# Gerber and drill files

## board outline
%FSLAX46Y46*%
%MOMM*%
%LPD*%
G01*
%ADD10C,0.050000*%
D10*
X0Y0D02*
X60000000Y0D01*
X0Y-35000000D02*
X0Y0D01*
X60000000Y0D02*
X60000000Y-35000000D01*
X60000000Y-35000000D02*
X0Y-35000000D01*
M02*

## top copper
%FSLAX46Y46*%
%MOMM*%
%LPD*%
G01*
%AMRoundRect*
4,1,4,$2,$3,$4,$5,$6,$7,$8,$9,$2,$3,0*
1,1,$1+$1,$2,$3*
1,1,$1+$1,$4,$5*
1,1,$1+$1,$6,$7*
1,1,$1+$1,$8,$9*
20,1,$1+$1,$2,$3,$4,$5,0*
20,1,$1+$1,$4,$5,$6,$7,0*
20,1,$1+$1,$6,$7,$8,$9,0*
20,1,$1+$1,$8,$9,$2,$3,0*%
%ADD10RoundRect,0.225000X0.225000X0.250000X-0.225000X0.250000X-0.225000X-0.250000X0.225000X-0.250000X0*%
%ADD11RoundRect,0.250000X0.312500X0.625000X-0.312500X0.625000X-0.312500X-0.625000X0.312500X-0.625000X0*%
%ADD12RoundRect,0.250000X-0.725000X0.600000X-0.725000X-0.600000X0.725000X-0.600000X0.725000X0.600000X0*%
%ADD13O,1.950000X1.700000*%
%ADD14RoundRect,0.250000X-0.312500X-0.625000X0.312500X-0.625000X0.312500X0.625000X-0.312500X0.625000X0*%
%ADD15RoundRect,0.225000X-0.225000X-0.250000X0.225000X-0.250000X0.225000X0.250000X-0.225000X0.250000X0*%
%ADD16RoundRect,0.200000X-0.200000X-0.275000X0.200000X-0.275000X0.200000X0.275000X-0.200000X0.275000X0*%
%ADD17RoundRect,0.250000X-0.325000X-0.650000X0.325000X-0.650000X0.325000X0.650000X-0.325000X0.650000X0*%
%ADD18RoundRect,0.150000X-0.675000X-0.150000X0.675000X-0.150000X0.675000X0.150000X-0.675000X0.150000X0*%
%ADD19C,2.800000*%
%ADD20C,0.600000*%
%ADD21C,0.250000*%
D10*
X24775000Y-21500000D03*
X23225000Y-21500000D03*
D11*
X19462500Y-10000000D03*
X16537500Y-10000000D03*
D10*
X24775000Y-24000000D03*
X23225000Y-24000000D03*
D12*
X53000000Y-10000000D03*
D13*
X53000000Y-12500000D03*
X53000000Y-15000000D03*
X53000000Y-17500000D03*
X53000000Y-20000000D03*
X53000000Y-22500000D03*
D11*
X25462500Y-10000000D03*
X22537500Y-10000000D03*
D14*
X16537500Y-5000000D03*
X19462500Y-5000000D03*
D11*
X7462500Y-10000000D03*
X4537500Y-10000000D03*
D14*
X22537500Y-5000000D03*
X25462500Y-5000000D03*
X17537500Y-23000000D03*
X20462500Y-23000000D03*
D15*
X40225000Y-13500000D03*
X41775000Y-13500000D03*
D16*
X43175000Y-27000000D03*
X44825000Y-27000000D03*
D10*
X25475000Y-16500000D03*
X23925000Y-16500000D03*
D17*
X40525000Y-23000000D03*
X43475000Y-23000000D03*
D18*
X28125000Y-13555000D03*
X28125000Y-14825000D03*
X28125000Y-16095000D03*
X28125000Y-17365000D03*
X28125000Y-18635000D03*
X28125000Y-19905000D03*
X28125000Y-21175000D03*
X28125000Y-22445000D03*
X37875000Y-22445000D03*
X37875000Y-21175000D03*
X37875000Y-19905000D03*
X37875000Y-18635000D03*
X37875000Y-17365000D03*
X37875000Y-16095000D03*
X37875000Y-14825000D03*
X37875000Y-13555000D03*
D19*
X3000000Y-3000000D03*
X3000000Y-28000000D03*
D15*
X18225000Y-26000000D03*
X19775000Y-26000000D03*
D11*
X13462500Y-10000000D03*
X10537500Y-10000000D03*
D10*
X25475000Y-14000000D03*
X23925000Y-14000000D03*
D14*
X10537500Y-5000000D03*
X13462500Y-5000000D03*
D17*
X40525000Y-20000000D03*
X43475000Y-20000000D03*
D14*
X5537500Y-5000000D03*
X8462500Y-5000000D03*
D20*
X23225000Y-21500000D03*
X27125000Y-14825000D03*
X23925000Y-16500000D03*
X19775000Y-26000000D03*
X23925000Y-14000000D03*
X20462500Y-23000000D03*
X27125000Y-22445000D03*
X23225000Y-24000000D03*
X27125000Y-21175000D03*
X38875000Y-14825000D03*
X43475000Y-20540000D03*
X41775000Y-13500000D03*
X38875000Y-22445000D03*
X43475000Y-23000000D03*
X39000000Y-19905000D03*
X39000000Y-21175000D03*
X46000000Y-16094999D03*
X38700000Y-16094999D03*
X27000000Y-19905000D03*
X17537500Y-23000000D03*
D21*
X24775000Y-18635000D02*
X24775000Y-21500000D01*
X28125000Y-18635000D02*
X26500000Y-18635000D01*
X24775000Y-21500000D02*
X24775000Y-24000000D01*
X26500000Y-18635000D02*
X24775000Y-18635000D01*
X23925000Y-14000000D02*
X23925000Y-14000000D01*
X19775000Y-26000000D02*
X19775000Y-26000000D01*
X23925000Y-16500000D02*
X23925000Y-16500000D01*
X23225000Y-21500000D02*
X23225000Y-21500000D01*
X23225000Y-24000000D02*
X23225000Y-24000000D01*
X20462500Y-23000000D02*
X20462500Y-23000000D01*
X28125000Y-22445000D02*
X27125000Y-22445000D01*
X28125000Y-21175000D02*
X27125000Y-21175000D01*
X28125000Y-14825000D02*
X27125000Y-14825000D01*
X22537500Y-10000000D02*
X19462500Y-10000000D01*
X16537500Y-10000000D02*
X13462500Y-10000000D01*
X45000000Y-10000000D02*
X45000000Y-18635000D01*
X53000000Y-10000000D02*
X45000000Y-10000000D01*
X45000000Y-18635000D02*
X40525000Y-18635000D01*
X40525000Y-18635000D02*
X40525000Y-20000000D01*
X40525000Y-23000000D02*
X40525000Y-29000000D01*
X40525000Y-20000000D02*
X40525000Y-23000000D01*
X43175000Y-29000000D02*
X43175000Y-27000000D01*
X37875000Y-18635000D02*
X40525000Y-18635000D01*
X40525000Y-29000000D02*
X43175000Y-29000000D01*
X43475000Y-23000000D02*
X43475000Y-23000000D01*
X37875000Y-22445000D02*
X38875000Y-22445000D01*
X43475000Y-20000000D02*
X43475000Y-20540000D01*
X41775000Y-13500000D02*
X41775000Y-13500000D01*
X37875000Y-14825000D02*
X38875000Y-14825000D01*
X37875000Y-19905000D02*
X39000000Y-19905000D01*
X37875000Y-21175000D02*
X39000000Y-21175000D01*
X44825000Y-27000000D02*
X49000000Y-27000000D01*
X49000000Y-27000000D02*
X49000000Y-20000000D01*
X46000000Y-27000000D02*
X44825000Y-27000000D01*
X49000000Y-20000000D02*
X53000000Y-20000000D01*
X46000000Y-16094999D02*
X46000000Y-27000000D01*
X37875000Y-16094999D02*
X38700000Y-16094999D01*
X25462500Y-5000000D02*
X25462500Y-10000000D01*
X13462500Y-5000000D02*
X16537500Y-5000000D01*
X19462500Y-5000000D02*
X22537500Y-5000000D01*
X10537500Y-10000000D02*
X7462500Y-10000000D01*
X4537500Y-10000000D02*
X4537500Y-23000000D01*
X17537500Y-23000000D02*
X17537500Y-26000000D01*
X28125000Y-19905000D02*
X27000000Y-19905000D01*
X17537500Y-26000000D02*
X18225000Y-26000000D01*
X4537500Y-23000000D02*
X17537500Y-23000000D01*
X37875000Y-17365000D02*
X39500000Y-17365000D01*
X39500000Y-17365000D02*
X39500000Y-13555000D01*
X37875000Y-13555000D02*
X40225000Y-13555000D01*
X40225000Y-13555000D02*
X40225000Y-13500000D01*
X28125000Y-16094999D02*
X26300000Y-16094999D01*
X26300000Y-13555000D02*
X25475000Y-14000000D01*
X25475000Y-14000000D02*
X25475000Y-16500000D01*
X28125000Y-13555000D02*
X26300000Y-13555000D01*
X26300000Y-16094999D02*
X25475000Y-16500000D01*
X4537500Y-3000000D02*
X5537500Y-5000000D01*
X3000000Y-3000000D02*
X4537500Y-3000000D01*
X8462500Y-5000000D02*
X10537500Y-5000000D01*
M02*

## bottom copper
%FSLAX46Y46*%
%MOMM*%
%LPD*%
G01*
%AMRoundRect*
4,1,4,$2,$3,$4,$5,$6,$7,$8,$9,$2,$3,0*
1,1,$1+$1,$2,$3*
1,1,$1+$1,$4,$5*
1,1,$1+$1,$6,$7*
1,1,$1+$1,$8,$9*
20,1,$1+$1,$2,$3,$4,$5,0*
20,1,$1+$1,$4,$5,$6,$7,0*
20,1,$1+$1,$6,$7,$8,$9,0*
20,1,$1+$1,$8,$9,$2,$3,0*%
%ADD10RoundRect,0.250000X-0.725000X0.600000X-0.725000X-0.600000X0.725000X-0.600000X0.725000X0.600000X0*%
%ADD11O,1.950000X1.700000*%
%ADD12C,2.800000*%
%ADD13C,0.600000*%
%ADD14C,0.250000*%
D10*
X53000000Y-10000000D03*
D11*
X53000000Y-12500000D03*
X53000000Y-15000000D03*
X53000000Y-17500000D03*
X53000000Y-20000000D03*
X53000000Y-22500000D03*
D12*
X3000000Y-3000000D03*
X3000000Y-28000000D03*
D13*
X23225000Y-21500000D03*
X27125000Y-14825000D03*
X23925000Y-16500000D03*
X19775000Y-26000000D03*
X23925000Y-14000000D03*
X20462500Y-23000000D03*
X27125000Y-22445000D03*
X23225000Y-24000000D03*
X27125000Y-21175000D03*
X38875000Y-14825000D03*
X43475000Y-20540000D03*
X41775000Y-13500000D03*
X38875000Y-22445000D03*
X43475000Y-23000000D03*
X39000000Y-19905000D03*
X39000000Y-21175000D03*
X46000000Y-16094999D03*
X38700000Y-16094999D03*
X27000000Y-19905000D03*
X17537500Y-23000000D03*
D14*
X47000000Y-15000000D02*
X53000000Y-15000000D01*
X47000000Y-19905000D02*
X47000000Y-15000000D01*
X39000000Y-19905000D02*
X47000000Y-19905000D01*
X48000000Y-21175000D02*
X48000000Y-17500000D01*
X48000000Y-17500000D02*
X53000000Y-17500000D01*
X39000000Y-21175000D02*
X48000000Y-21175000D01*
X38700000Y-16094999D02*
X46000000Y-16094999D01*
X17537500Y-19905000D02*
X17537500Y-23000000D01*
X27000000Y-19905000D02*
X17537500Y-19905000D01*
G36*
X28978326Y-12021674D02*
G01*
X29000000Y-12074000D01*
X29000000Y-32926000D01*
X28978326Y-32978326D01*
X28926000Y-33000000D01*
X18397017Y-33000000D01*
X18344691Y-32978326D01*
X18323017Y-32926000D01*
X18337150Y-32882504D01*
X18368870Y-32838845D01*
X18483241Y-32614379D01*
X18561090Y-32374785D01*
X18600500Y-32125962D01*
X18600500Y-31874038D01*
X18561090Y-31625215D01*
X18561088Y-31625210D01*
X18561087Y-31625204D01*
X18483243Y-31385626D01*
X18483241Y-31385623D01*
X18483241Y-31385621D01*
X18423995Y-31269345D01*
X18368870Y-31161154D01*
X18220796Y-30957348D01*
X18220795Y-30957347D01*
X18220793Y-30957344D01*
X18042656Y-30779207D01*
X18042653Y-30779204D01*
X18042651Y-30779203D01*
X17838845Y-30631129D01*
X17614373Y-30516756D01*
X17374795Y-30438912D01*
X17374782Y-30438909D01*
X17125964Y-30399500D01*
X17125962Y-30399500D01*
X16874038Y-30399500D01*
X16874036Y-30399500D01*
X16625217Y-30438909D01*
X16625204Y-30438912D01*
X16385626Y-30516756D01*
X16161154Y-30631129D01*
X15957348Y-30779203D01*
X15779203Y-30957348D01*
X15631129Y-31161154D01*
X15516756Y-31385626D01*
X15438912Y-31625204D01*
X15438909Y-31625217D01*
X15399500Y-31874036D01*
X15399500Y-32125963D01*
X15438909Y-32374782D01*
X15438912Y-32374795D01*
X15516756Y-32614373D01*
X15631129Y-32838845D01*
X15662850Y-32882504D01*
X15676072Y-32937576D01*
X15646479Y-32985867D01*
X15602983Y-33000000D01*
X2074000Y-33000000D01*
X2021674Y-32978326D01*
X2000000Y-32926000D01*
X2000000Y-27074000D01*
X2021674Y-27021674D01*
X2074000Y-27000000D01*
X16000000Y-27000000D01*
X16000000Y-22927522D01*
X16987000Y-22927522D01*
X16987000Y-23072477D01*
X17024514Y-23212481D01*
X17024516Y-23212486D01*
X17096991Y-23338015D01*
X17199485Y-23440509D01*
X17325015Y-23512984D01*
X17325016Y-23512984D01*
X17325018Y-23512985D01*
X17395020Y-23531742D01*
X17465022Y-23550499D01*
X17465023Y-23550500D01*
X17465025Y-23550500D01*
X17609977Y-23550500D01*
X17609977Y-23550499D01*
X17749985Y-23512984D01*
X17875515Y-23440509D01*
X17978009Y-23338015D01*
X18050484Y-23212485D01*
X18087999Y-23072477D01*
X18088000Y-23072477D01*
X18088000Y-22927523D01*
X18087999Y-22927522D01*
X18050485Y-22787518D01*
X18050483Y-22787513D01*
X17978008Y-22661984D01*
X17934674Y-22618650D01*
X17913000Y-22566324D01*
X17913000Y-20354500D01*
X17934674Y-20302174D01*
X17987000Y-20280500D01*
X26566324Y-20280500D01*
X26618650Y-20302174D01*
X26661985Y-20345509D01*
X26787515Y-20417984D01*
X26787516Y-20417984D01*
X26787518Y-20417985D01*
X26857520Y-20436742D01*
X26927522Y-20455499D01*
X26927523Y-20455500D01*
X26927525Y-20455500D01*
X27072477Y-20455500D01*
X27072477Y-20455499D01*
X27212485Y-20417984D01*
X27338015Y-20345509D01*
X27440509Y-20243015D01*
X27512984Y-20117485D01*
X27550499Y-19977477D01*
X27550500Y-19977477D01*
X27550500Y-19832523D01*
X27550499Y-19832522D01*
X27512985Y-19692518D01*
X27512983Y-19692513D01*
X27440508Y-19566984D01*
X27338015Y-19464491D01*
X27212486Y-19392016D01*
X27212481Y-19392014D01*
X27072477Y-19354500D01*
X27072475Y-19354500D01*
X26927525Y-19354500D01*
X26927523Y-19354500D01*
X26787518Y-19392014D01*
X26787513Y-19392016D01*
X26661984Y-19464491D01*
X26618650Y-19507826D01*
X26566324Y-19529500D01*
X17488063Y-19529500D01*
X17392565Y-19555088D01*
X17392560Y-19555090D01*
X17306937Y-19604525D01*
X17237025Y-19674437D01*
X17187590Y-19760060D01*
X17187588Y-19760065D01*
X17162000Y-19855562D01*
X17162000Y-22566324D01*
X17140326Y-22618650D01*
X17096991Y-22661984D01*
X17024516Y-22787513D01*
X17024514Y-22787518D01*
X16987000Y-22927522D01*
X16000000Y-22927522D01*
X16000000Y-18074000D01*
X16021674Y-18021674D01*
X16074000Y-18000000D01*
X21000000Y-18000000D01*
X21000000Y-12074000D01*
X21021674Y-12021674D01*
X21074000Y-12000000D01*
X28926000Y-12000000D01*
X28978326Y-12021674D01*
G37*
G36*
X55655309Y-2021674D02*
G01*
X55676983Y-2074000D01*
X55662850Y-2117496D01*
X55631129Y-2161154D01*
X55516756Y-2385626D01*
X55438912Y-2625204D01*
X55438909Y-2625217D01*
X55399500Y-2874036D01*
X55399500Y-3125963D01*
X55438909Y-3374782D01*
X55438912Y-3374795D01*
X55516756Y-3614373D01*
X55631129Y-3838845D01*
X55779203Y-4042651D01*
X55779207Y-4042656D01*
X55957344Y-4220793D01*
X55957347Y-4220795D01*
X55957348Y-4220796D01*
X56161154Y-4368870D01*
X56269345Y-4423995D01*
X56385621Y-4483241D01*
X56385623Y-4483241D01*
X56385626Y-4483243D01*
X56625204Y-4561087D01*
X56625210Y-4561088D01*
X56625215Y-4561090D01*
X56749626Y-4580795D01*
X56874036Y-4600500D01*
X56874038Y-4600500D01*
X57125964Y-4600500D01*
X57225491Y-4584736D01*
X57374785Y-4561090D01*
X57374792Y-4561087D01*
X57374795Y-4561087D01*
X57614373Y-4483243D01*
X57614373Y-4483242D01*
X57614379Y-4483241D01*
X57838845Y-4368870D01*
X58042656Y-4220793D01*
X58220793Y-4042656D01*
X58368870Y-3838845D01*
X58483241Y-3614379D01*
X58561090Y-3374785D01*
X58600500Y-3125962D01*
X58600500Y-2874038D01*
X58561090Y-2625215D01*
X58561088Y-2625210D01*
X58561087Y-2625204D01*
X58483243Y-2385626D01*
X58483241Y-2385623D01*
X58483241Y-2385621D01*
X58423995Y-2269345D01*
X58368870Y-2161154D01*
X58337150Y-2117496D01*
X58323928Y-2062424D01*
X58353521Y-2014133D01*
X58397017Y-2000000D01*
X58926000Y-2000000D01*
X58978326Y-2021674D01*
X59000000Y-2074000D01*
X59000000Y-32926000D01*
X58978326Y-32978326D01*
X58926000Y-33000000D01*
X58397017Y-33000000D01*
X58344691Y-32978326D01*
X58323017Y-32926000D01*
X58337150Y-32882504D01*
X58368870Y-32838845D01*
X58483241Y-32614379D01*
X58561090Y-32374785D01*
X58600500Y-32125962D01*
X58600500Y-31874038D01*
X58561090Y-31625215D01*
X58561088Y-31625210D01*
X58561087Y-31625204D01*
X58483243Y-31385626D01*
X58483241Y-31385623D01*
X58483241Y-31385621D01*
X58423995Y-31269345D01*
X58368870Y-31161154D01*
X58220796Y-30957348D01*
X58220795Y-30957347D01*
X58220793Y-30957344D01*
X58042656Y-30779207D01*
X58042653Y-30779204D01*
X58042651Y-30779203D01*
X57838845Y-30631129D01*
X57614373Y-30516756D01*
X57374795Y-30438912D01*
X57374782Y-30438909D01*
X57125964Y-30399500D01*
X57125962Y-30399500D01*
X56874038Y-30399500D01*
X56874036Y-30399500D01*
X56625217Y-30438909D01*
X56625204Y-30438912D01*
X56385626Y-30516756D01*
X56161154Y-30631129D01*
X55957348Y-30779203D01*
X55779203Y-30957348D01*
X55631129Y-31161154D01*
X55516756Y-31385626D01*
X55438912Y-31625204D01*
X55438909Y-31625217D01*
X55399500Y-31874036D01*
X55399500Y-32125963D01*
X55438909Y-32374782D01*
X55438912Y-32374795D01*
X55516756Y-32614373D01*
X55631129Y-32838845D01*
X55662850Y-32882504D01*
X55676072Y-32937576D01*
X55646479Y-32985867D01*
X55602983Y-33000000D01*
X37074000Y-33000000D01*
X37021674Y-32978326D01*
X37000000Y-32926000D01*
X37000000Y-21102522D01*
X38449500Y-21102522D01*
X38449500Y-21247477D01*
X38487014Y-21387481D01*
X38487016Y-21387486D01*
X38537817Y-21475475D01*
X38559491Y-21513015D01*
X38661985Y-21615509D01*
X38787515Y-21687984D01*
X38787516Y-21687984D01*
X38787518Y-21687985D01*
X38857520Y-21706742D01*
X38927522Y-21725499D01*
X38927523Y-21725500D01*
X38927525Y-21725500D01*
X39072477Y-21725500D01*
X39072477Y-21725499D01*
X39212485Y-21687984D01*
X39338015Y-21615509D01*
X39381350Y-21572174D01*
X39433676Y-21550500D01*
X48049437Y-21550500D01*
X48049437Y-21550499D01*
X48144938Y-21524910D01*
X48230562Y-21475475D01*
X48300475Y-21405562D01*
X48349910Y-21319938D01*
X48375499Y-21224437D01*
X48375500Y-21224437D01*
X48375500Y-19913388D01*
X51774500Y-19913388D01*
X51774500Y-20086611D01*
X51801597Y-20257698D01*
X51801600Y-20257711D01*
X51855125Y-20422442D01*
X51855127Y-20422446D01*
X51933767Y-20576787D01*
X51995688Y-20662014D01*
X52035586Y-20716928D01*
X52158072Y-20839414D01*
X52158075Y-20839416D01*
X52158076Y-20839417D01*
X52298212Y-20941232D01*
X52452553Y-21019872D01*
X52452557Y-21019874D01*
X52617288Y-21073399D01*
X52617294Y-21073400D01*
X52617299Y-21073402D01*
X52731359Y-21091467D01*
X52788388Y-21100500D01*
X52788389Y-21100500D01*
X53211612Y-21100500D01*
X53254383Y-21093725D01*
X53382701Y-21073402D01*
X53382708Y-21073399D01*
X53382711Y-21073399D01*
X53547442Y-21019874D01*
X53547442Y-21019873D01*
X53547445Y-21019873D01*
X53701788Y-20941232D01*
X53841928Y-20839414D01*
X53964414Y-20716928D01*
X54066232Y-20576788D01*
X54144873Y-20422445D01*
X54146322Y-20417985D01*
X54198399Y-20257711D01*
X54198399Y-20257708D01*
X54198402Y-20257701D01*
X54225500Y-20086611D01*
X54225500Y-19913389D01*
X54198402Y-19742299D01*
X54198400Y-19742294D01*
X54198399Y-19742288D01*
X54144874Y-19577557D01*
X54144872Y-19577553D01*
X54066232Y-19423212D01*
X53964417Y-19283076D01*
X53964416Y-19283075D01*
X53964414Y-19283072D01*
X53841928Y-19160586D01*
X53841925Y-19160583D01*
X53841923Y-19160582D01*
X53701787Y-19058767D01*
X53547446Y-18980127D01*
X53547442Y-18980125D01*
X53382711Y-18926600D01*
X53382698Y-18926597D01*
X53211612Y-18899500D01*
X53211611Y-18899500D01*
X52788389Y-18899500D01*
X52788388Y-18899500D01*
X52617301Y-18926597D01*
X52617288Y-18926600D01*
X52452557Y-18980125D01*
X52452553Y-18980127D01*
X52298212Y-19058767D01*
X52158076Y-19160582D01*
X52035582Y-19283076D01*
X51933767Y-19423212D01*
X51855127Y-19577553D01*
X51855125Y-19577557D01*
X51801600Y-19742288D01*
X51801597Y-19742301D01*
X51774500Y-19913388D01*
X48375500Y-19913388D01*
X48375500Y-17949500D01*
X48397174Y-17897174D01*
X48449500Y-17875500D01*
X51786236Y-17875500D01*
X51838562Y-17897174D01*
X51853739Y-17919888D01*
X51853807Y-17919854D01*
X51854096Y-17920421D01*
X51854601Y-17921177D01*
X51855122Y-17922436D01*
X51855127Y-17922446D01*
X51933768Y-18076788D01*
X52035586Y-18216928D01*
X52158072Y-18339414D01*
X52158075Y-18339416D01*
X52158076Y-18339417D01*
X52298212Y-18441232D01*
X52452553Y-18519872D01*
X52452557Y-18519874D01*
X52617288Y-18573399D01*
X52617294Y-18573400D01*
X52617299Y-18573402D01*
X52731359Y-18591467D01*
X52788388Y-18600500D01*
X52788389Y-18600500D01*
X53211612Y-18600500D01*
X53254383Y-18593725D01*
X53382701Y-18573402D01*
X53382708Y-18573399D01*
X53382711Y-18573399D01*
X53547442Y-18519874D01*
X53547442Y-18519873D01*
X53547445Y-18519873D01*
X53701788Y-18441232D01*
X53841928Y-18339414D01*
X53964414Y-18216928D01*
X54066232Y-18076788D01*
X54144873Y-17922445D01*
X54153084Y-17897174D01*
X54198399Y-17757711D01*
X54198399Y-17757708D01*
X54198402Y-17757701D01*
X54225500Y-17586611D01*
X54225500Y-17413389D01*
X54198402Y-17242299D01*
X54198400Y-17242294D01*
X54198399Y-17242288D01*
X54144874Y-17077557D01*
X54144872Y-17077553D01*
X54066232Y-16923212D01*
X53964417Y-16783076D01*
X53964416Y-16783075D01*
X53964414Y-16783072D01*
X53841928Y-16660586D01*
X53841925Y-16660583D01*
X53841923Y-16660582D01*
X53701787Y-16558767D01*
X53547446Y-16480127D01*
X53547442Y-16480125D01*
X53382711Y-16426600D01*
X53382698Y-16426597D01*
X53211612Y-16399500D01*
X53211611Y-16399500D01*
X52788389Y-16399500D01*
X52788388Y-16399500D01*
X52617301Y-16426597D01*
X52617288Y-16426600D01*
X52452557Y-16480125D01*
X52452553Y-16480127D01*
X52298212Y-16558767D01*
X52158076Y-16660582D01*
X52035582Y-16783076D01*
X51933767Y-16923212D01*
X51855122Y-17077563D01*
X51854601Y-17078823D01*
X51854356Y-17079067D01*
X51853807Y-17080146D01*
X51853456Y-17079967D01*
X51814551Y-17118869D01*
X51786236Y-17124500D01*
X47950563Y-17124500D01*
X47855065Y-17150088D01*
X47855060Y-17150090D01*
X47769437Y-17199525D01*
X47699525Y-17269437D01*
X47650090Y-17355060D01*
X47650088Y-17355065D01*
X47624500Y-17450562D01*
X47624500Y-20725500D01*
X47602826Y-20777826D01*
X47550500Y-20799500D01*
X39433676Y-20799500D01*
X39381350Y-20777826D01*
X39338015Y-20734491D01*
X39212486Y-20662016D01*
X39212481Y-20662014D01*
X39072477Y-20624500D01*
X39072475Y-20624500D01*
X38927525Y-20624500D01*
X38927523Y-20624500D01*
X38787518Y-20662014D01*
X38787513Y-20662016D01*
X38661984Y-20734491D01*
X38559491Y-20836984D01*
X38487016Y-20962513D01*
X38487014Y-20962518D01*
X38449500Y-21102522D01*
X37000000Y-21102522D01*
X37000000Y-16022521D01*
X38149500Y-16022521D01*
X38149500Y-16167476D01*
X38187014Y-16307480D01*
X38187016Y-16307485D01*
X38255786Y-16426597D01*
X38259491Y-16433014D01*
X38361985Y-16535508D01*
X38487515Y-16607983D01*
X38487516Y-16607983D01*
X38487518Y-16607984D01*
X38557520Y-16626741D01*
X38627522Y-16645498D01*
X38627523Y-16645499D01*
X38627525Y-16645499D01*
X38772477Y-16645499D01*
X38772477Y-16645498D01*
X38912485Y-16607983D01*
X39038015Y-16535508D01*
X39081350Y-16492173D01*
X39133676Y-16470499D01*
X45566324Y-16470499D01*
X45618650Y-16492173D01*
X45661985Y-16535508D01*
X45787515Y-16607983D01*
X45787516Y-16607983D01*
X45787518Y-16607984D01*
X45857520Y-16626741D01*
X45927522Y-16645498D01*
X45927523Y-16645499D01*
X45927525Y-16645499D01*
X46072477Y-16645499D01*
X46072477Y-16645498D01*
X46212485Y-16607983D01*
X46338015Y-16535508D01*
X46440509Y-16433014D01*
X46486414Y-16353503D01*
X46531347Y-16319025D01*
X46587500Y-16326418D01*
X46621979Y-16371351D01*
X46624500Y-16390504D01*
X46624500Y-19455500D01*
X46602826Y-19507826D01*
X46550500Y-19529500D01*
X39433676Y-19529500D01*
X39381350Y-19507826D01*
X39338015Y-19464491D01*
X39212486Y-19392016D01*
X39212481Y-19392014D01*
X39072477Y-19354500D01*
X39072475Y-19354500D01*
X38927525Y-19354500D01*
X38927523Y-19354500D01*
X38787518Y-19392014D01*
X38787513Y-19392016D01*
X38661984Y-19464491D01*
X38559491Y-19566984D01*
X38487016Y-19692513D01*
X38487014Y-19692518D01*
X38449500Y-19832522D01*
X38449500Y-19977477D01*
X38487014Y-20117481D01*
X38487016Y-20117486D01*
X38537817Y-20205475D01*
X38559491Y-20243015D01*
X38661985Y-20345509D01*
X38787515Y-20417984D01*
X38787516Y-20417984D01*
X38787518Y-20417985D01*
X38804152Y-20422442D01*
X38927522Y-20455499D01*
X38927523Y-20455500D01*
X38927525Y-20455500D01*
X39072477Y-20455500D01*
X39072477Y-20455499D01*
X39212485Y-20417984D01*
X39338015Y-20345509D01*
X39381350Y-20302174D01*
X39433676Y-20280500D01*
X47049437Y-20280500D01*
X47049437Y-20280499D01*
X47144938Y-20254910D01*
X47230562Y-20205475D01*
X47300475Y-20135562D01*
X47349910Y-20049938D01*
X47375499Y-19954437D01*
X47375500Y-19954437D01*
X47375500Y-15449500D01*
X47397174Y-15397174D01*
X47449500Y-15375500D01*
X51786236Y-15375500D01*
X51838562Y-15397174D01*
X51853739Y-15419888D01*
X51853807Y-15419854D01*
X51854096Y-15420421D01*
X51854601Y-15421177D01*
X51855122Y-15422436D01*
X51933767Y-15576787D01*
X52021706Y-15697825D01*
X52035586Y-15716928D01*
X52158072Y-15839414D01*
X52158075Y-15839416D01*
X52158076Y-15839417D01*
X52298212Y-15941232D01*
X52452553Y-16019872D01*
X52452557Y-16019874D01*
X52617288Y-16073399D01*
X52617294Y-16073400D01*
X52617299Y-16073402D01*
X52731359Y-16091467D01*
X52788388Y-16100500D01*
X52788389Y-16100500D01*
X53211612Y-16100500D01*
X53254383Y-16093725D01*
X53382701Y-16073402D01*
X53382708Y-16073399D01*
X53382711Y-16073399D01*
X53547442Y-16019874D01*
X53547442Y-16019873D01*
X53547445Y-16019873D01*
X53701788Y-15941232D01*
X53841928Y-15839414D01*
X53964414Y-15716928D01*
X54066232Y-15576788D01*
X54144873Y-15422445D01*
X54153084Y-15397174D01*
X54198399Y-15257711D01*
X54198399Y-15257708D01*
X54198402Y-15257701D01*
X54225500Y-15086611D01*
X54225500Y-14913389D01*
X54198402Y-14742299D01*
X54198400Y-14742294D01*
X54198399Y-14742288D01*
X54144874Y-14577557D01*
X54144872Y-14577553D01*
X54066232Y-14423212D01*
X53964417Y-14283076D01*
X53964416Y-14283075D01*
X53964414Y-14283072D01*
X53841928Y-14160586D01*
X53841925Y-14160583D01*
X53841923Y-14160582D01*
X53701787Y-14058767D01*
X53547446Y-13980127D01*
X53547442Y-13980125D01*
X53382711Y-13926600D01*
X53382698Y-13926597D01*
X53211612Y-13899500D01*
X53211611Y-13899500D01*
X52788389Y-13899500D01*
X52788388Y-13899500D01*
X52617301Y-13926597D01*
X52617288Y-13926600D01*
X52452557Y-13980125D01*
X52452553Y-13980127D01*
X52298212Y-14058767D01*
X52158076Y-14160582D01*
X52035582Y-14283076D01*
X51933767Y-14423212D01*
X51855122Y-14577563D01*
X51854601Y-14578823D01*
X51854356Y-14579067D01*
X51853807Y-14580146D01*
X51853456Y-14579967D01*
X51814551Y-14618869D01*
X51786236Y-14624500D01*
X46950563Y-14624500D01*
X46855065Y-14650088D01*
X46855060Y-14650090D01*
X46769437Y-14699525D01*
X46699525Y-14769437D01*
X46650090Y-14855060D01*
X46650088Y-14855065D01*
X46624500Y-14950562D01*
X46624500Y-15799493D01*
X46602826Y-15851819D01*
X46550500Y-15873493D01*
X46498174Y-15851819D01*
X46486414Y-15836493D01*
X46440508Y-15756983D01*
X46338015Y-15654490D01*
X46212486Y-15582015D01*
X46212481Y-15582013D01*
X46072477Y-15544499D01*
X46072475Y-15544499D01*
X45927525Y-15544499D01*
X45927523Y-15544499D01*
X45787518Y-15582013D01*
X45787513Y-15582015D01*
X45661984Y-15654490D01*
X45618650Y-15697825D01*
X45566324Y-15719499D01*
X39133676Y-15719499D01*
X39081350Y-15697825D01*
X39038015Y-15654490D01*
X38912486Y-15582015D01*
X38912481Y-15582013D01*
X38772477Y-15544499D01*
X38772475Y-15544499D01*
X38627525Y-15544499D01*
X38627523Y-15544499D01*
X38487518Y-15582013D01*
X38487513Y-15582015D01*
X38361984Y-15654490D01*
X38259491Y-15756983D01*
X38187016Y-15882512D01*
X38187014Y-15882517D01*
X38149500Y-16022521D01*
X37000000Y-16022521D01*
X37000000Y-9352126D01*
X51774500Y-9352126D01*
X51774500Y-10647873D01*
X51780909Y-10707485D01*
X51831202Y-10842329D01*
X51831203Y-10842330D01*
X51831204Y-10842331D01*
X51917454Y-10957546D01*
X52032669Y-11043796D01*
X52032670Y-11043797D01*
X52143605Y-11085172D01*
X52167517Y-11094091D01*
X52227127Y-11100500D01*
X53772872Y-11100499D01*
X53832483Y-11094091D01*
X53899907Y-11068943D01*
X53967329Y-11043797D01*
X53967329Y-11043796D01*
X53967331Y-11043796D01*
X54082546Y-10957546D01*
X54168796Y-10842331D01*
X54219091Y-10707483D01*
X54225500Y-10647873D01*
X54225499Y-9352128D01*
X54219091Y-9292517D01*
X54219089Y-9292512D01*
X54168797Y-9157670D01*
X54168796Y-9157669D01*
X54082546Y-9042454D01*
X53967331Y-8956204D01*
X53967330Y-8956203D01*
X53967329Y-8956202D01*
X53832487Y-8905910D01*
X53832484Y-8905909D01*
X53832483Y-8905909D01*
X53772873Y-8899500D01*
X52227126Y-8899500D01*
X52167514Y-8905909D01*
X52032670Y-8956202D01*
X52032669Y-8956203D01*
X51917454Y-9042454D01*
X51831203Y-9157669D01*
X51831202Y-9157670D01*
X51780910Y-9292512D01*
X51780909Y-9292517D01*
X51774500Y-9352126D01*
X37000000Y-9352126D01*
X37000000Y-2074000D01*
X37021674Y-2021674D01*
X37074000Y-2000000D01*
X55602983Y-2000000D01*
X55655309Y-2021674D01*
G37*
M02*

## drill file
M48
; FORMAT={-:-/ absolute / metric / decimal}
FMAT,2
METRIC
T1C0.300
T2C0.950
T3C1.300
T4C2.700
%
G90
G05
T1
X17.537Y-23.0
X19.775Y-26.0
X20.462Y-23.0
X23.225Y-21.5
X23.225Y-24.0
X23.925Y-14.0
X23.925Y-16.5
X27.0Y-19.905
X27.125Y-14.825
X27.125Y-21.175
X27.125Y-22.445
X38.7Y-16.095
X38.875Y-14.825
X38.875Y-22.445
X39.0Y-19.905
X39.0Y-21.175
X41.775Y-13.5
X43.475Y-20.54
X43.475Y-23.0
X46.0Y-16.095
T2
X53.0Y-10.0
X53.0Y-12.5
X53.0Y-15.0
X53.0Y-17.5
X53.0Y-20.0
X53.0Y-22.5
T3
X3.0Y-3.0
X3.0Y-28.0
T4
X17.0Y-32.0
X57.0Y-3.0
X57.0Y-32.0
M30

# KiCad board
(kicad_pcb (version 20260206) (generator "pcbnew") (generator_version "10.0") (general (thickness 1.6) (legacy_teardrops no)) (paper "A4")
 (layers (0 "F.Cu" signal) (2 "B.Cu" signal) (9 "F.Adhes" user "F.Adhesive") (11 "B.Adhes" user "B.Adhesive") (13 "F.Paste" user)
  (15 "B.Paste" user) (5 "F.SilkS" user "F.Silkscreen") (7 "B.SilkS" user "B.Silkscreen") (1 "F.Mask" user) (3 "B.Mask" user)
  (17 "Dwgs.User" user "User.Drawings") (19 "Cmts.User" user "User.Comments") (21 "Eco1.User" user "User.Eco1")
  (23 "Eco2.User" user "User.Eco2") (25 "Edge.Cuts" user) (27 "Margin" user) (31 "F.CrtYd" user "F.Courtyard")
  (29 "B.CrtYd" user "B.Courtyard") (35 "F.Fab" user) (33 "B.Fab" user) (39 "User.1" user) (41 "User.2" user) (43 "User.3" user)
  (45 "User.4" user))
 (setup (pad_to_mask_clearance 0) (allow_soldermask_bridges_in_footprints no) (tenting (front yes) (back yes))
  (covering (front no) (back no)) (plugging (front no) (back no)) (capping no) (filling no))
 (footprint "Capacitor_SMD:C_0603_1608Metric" (layer "F.Cu") (at 24 21.5 180)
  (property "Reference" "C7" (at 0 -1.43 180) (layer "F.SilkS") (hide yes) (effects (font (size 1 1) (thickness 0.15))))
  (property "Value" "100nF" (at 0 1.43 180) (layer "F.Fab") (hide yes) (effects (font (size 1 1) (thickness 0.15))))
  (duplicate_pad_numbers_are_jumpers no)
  (pad "1" smd roundrect (at -0.775 0 180) (size 0.9 0.95) (layers "F.Cu" "F.Mask" "F.Paste") (roundrect_rratio 0.25) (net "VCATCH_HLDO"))
  (pad "2" smd roundrect (at 0.775 0 180) (size 0.9 0.95) (layers "F.Cu" "F.Mask" "F.Paste") (roundrect_rratio 0.25) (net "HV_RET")))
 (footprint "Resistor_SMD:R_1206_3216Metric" (layer "F.Cu") (at 18 10 180)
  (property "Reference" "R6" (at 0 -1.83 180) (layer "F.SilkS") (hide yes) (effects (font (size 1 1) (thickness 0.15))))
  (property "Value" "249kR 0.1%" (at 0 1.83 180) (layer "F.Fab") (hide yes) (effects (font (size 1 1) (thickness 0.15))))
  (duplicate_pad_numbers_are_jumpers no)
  (pad "1" smd roundrect (at -1.4625 0 180) (size 1.125 1.75) (layers "F.Cu" "F.Mask" "F.Paste") (roundrect_rratio 0.222222)
   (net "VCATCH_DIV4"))
  (pad "2" smd roundrect (at 1.4625 0 180) (size 1.125 1.75) (layers "F.Cu" "F.Mask" "F.Paste") (roundrect_rratio 0.222222)
   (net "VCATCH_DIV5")))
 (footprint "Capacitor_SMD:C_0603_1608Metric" (layer "F.Cu") (at 24 24 180)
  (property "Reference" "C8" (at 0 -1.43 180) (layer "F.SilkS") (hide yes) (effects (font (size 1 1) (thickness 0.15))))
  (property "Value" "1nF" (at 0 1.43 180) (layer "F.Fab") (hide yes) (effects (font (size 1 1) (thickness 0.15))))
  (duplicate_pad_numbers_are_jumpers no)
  (pad "1" smd roundrect (at -0.775 0 180) (size 0.9 0.95) (layers "F.Cu" "F.Mask" "F.Paste") (roundrect_rratio 0.25) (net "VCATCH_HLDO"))
  (pad "2" smd roundrect (at 0.775 0 180) (size 0.9 0.95) (layers "F.Cu" "F.Mask" "F.Paste") (roundrect_rratio 0.25) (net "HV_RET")))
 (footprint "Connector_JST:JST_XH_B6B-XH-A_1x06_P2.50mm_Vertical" (layer "F.Cu") (at 53 10 -90)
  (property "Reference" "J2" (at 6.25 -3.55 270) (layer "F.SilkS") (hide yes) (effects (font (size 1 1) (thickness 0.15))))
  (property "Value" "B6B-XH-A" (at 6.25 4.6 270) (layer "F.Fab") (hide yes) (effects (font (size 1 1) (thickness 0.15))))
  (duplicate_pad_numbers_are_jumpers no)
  (pad "1" thru_hole roundrect (at 0 0 270) (size 1.7 1.95) (drill 0.95) (layers "*.Cu" "*.Mask") (remove_unused_layers no)
   (roundrect_rratio 0.147059) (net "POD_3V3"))
  (pad "2" thru_hole oval (at 2.5 0 270) (size 1.7 1.95) (drill 0.95) (layers "*.Cu" "*.Mask") (remove_unused_layers no) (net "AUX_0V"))
  (pad "3" thru_hole oval (at 5 0 270) (size 1.7 1.95) (drill 0.95) (layers "*.Cu" "*.Mask") (remove_unused_layers no) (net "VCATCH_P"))
  (pad "4" thru_hole oval (at 7.5 0 270) (size 1.7 1.95) (drill 0.95) (layers "*.Cu" "*.Mask") (remove_unused_layers no) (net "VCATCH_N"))
  (pad "5" thru_hole oval (at 10 0 270) (size 1.7 1.95) (drill 0.95) (layers "*.Cu" "*.Mask") (remove_unused_layers no)
   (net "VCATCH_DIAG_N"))
  (pad "6" thru_hole oval (at 12.5 0 270) (size 1.7 1.95) (drill 0.95) (layers "*.Cu" "*.Mask") (remove_unused_layers no) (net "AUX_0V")))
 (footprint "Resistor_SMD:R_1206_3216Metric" (layer "F.Cu") (at 24 10 180)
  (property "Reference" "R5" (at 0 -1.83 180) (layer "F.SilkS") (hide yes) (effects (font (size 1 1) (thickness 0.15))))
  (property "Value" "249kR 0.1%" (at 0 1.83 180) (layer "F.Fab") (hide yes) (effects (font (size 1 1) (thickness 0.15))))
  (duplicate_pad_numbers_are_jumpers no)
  (pad "1" smd roundrect (at -1.4625 0 180) (size 1.125 1.75) (layers "F.Cu" "F.Mask" "F.Paste") (roundrect_rratio 0.222222)
   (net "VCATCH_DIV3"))
  (pad "2" smd roundrect (at 1.4625 0 180) (size 1.125 1.75) (layers "F.Cu" "F.Mask" "F.Paste") (roundrect_rratio 0.222222)
   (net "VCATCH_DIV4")))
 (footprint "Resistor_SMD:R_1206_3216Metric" (layer "F.Cu") (at 18 5)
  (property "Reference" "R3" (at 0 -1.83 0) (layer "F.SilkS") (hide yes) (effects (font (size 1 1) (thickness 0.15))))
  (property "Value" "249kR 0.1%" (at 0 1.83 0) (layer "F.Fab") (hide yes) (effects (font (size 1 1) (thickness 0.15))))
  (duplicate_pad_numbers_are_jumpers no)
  (pad "1" smd roundrect (at -1.4625 0) (size 1.125 1.75) (layers "F.Cu" "F.Mask" "F.Paste") (roundrect_rratio 0.222222) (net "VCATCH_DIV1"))
  (pad "2" smd roundrect (at 1.4625 0) (size 1.125 1.75) (layers "F.Cu" "F.Mask" "F.Paste") (roundrect_rratio 0.222222) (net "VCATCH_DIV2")))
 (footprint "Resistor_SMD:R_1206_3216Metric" (layer "F.Cu") (at 6 10 180)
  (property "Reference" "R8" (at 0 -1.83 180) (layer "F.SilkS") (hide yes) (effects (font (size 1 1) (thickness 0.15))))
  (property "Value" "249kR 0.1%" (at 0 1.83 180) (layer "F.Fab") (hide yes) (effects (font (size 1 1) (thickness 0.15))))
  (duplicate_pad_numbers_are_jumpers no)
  (pad "1" smd roundrect (at -1.4625 0 180) (size 1.125 1.75) (layers "F.Cu" "F.Mask" "F.Paste") (roundrect_rratio 0.222222)
   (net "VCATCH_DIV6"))
  (pad "2" smd roundrect (at 1.4625 0 180) (size 1.125 1.75) (layers "F.Cu" "F.Mask" "F.Paste") (roundrect_rratio 0.222222)
   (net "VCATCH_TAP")))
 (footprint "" (layer "F.Cu") (at 17 32)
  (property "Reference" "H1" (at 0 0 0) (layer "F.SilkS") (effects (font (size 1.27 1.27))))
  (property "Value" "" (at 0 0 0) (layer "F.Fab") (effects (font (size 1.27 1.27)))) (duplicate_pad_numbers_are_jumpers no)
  (pad "" np_thru_hole circle (at 0 0) (size 2.7 2.7) (drill 2.7) (layers "*.Cu")))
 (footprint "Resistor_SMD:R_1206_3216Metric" (layer "F.Cu") (at 24 5)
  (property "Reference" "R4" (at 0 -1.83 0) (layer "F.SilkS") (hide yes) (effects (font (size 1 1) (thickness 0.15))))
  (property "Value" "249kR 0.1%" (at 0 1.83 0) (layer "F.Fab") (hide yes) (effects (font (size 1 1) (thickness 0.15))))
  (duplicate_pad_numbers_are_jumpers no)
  (pad "1" smd roundrect (at -1.4625 0) (size 1.125 1.75) (layers "F.Cu" "F.Mask" "F.Paste") (roundrect_rratio 0.222222) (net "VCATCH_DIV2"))
  (pad "2" smd roundrect (at 1.4625 0) (size 1.125 1.75) (layers "F.Cu" "F.Mask" "F.Paste") (roundrect_rratio 0.222222) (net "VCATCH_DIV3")))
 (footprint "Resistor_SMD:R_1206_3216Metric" (layer "F.Cu") (at 19 23)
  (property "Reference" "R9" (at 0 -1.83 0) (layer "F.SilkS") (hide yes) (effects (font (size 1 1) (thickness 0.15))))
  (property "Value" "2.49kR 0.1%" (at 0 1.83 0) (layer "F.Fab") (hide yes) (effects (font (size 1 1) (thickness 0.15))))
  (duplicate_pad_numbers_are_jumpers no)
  (pad "1" smd roundrect (at -1.4625 0) (size 1.125 1.75) (layers "F.Cu" "F.Mask" "F.Paste") (roundrect_rratio 0.222222) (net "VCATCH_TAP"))
  (pad "2" smd roundrect (at 1.4625 0) (size 1.125 1.75) (layers "F.Cu" "F.Mask" "F.Paste") (roundrect_rratio 0.222222) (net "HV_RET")))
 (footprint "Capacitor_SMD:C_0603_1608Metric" (layer "F.Cu") (at 41 13.5)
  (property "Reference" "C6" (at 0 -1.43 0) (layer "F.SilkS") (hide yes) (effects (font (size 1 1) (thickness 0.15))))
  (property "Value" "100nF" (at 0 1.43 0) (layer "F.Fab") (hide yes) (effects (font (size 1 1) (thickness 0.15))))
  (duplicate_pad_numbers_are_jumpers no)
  (pad "1" smd roundrect (at -0.775 0) (size 0.9 0.95) (layers "F.Cu" "F.Mask" "F.Paste") (roundrect_rratio 0.25) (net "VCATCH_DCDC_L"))
  (pad "2" smd roundrect (at 0.775 0) (size 0.9 0.95) (layers "F.Cu" "F.Mask" "F.Paste") (roundrect_rratio 0.25) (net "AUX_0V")))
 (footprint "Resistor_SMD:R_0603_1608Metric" (layer "F.Cu") (at 44 27)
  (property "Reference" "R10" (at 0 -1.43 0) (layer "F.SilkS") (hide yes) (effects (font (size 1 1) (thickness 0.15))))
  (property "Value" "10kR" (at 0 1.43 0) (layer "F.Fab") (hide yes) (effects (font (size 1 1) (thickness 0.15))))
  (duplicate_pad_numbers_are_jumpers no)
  (pad "1" smd roundrect (at -0.825 0) (size 0.8 0.95) (layers "F.Cu" "F.Mask" "F.Paste") (roundrect_rratio 0.25) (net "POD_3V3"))
  (pad "2" smd roundrect (at 0.825 0) (size 0.8 0.95) (layers "F.Cu" "F.Mask" "F.Paste") (roundrect_rratio 0.25) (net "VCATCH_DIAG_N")))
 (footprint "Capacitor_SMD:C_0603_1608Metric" (layer "F.Cu") (at 24.7 16.5 180)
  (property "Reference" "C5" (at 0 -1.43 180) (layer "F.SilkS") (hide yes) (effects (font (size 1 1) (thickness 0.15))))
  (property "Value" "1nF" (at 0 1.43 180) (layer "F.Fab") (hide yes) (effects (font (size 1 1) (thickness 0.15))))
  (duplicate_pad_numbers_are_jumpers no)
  (pad "1" smd roundrect (at -0.775 0 180) (size 0.9 0.95) (layers "F.Cu" "F.Mask" "F.Paste") (roundrect_rratio 0.25) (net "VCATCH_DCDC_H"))
  (pad "2" smd roundrect (at 0.775 0 180) (size 0.9 0.95) (layers "F.Cu" "F.Mask" "F.Paste") (roundrect_rratio 0.25) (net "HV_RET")))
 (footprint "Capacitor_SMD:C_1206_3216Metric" (layer "F.Cu") (at 42 23)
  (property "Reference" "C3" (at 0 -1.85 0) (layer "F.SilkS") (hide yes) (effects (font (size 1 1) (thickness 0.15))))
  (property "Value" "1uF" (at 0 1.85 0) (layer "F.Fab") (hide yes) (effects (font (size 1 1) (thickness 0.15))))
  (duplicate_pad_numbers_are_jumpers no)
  (pad "1" smd roundrect (at -1.475 0) (size 1.15 1.8) (layers "F.Cu" "F.Mask" "F.Paste") (roundrect_rratio 0.217391) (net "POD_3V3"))
  (pad "2" smd roundrect (at 1.475 0) (size 1.15 1.8) (layers "F.Cu" "F.Mask" "F.Paste") (roundrect_rratio 0.217391) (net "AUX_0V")))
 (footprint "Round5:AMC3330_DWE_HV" (layer "F.Cu") (at 33 18)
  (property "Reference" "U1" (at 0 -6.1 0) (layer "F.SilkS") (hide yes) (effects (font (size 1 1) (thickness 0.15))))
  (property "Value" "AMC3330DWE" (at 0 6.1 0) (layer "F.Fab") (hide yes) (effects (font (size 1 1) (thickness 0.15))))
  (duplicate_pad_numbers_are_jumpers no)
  (pad "1" smd roundrect (at -4.875 -4.445) (size 1.65 0.6) (layers "F.Cu" "F.Mask" "F.Paste") (roundrect_rratio 0.25) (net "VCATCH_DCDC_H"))
  (pad "2" smd roundrect (at -4.875 -3.175) (size 1.65 0.6) (layers "F.Cu" "F.Mask" "F.Paste") (roundrect_rratio 0.25) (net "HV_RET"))
  (pad "3" smd roundrect (at -4.875 -1.905) (size 1.65 0.6) (layers "F.Cu" "F.Mask" "F.Paste") (roundrect_rratio 0.25) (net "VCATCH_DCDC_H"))
  (pad "4" smd roundrect (at -4.875 -0.635) (size 1.65 0.6) (layers "F.Cu" "F.Mask" "F.Paste") (roundrect_rratio 0.25)
   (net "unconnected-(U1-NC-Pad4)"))
  (pad "5" smd roundrect (at -4.875 0.635) (size 1.65 0.6) (layers "F.Cu" "F.Mask" "F.Paste") (roundrect_rratio 0.25) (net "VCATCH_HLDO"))
  (pad "6" smd roundrect (at -4.875 1.905) (size 1.65 0.6) (layers "F.Cu" "F.Mask" "F.Paste") (roundrect_rratio 0.25) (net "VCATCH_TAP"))
  (pad "7" smd roundrect (at -4.875 3.175) (size 1.65 0.6) (layers "F.Cu" "F.Mask" "F.Paste") (roundrect_rratio 0.25) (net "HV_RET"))
  (pad "8" smd roundrect (at -4.875 4.445) (size 1.65 0.6) (layers "F.Cu" "F.Mask" "F.Paste") (roundrect_rratio 0.25) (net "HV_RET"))
  (pad "9" smd roundrect (at 4.875 4.445) (size 1.65 0.6) (layers "F.Cu" "F.Mask" "F.Paste") (roundrect_rratio 0.25) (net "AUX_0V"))
  (pad "10" smd roundrect (at 4.875 3.175) (size 1.65 0.6) (layers "F.Cu" "F.Mask" "F.Paste") (roundrect_rratio 0.25) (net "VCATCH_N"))
  (pad "11" smd roundrect (at 4.875 1.905) (size 1.65 0.6) (layers "F.Cu" "F.Mask" "F.Paste") (roundrect_rratio 0.25) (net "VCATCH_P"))
  (pad "12" smd roundrect (at 4.875 0.635) (size 1.65 0.6) (layers "F.Cu" "F.Mask" "F.Paste") (roundrect_rratio 0.25) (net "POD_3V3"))
  (pad "13" smd roundrect (at 4.875 -0.635) (size 1.65 0.6) (layers "F.Cu" "F.Mask" "F.Paste") (roundrect_rratio 0.25) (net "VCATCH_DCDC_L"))
  (pad "14" smd roundrect (at 4.875 -1.905) (size 1.65 0.6) (layers "F.Cu" "F.Mask" "F.Paste") (roundrect_rratio 0.25) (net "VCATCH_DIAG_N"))
  (pad "15" smd roundrect (at 4.875 -3.175) (size 1.65 0.6) (layers "F.Cu" "F.Mask" "F.Paste") (roundrect_rratio 0.25) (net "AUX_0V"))
  (pad "16" smd roundrect (at 4.875 -4.445) (size 1.65 0.6) (layers "F.Cu" "F.Mask" "F.Paste") (roundrect_rratio 0.25) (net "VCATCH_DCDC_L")))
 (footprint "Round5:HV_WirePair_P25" (layer "F.Cu") (at 3 3)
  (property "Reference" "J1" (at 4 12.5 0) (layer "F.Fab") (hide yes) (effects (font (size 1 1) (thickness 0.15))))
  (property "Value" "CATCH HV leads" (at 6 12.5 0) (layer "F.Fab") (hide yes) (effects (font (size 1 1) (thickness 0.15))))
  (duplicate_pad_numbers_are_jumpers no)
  (pad "1" thru_hole circle (at 0 0) (size 2.8 2.8) (drill 1.3) (layers "*.Cu" "*.Mask") (remove_unused_layers no) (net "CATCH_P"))
  (pad "2" thru_hole circle (at 0 25) (size 2.8 2.8) (drill 1.3) (layers "*.Cu" "*.Mask") (remove_unused_layers no) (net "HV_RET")))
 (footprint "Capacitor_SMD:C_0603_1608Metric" (layer "F.Cu") (at 19 26)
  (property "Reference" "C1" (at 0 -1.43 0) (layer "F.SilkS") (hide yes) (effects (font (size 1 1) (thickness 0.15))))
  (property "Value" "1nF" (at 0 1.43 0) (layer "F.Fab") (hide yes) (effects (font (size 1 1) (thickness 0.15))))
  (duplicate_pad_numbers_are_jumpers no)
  (pad "1" smd roundrect (at -0.775 0) (size 0.9 0.95) (layers "F.Cu" "F.Mask" "F.Paste") (roundrect_rratio 0.25) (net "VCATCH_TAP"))
  (pad "2" smd roundrect (at 0.775 0) (size 0.9 0.95) (layers "F.Cu" "F.Mask" "F.Paste") (roundrect_rratio 0.25) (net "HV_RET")))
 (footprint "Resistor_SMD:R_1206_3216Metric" (layer "F.Cu") (at 12 10 180)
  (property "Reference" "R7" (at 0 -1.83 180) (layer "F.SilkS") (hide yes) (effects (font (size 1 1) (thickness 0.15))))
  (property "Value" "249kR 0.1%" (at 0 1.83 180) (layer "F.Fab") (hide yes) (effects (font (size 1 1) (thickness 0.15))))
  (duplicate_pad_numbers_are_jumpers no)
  (pad "1" smd roundrect (at -1.4625 0 180) (size 1.125 1.75) (layers "F.Cu" "F.Mask" "F.Paste") (roundrect_rratio 0.222222)
   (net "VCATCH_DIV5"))
  (pad "2" smd roundrect (at 1.4625 0 180) (size 1.125 1.75) (layers "F.Cu" "F.Mask" "F.Paste") (roundrect_rratio 0.222222)
   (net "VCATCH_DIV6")))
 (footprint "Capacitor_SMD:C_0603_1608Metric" (layer "F.Cu") (at 24.7 14 180)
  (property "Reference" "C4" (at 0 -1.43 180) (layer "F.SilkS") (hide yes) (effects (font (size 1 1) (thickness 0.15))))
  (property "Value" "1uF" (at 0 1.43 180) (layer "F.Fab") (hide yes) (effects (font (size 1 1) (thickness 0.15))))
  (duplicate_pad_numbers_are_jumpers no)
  (pad "1" smd roundrect (at -0.775 0 180) (size 0.9 0.95) (layers "F.Cu" "F.Mask" "F.Paste") (roundrect_rratio 0.25) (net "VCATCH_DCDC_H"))
  (pad "2" smd roundrect (at 0.775 0 180) (size 0.9 0.95) (layers "F.Cu" "F.Mask" "F.Paste") (roundrect_rratio 0.25) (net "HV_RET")))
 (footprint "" (layer "F.Cu") (at 57 32)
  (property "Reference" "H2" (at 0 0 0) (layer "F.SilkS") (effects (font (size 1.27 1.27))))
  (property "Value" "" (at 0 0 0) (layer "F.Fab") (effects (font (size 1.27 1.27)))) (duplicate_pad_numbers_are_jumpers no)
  (pad "" np_thru_hole circle (at 0 0) (size 2.7 2.7) (drill 2.7) (layers "*.Cu")))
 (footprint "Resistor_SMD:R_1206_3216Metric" (layer "F.Cu") (at 12 5)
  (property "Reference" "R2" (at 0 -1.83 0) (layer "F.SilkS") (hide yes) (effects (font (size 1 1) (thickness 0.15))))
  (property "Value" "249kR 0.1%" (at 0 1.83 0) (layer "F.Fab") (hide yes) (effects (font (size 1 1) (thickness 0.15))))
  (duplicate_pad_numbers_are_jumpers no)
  (pad "1" smd roundrect (at -1.4625 0) (size 1.125 1.75) (layers "F.Cu" "F.Mask" "F.Paste") (roundrect_rratio 0.222222) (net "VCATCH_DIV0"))
  (pad "2" smd roundrect (at 1.4625 0) (size 1.125 1.75) (layers "F.Cu" "F.Mask" "F.Paste") (roundrect_rratio 0.222222) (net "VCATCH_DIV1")))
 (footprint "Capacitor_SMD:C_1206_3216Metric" (layer "F.Cu") (at 42 20)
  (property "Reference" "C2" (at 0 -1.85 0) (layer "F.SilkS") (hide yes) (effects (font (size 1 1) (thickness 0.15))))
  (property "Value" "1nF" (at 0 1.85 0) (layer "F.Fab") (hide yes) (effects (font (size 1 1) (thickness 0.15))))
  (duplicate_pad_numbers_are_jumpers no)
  (pad "1" smd roundrect (at -1.475 0) (size 1.15 1.8) (layers "F.Cu" "F.Mask" "F.Paste") (roundrect_rratio 0.217391) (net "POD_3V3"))
  (pad "2" smd roundrect (at 1.475 0) (size 1.15 1.8) (layers "F.Cu" "F.Mask" "F.Paste") (roundrect_rratio 0.217391) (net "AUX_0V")))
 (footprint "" (layer "F.Cu") (at 57 3)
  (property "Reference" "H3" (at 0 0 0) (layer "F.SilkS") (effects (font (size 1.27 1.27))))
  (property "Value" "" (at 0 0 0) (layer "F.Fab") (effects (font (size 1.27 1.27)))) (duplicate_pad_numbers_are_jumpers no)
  (pad "" np_thru_hole circle (at 0 0) (size 2.7 2.7) (drill 2.7) (layers "*.Cu")))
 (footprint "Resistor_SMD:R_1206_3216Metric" (layer "F.Cu") (at 7 5)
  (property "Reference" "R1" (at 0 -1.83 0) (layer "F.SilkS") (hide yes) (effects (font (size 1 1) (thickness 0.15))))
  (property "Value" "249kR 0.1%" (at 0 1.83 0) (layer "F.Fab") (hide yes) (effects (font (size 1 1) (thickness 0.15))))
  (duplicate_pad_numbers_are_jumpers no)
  (pad "1" smd roundrect (at -1.4625 0) (size 1.125 1.75) (layers "F.Cu" "F.Mask" "F.Paste") (roundrect_rratio 0.222222) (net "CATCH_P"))
  (pad "2" smd roundrect (at 1.4625 0) (size 1.125 1.75) (layers "F.Cu" "F.Mask" "F.Paste") (roundrect_rratio 0.222222) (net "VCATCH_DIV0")))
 (gr_line (start 0 0) (end 60 0) (stroke (width 0.05) (type default)) (layer "Edge.Cuts"))
 (gr_line (start 0 35) (end 0 0) (stroke (width 0.05) (type default)) (layer "Edge.Cuts"))
 (gr_line (start 60 0) (end 60 35) (stroke (width 0.05) (type default)) (layer "Edge.Cuts"))
 (gr_line (start 60 35) (end 0 35) (stroke (width 0.05) (type default)) (layer "Edge.Cuts"))
 (segment (start 24.775 18.635) (end 24.775 21.5) (width 0.25) (layer "F.Cu") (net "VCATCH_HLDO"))
 (segment (start 28.125 18.635) (end 26.5 18.635) (width 0.25) (layer "F.Cu") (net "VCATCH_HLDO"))
 (segment (start 24.775 21.5) (end 24.775 24) (width 0.25) (layer "F.Cu") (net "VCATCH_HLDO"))
 (segment (start 26.5 18.635) (end 24.775 18.635) (width 0.25) (layer "F.Cu") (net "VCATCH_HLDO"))
 (segment (start 23.925 14) (end 23.925 14) (width 0.25) (layer "F.Cu") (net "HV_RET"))
 (segment (start 19.775 26) (end 19.775 26) (width 0.25) (layer "F.Cu") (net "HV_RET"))
 (segment (start 23.925 16.5) (end 23.925 16.5) (width 0.25) (layer "F.Cu") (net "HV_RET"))
 (segment (start 23.225 21.5) (end 23.225 21.5) (width 0.25) (layer "F.Cu") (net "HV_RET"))
 (segment (start 23.225 24) (end 23.225 24) (width 0.25) (layer "F.Cu") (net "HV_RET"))
 (segment (start 20.4625 23) (end 20.4625 23) (width 0.25) (layer "F.Cu") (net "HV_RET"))
 (segment (start 28.125 22.445) (end 27.125 22.445) (width 0.25) (layer "F.Cu") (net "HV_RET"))
 (segment (start 28.125 21.175) (end 27.125 21.175) (width 0.25) (layer "F.Cu") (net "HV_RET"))
 (segment (start 28.125 14.825) (end 27.125 14.825) (width 0.25) (layer "F.Cu") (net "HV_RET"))
 (via (at 23.225 21.5) (size 0.6) (drill 0.3) (layers "F.Cu" "B.Cu") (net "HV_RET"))
 (via (at 27.125 14.825) (size 0.6) (drill 0.3) (layers "F.Cu" "B.Cu") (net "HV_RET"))
 (via (at 23.925 16.5) (size 0.6) (drill 0.3) (layers "F.Cu" "B.Cu") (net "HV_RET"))
 (via (at 19.775 26) (size 0.6) (drill 0.3) (layers "F.Cu" "B.Cu") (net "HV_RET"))
 (via (at 23.925 14) (size 0.6) (drill 0.3) (layers "F.Cu" "B.Cu") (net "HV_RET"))
 (via (at 20.4625 23) (size 0.6) (drill 0.3) (layers "F.Cu" "B.Cu") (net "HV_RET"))
 (via (at 27.125 22.445) (size 0.6) (drill 0.3) (layers "F.Cu" "B.Cu") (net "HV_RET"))
 (via (at 23.225 24) (size 0.6) (drill 0.3) (layers "F.Cu" "B.Cu") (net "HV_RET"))
 (via (at 27.125 21.175) (size 0.6) (drill 0.3) (layers "F.Cu" "B.Cu") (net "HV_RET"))
 (segment (start 22.5375 10) (end 19.4625 10) (width 0.25) (layer "F.Cu") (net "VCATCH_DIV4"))
 (segment (start 16.5375 10) (end 13.4625 10) (width 0.25) (layer "F.Cu") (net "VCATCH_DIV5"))
 (segment (start 45 10) (end 45 18.635) (width 0.25) (layer "F.Cu") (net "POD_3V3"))
 (segment (start 53 10) (end 45 10) (width 0.25) (layer "F.Cu") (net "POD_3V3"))
 (segment (start 45 18.635) (end 40.525 18.635) (width 0.25) (layer "F.Cu") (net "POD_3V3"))
 (segment (start 40.525 18.635) (end 40.525 20) (width 0.25) (layer "F.Cu") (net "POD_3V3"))
 (segment (start 40.525 23) (end 40.525 29) (width 0.25) (layer "F.Cu") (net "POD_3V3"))
 (segment (start 40.525 20) (end 40.525 23) (width 0.25) (layer "F.Cu") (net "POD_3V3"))
 (segment (start 43.175 29) (end 43.175 27) (width 0.25) (layer "F.Cu") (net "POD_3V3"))
 (segment (start 37.875 18.635) (end 40.525 18.635) (width 0.25) (layer "F.Cu") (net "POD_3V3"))
 (segment (start 40.525 29) (end 43.175 29) (width 0.25) (layer "F.Cu") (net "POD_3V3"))
 (segment (start 43.475 23) (end 43.475 23) (width 0.25) (layer "F.Cu") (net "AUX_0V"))
 (segment (start 37.875 22.445) (end 38.875 22.445) (width 0.25) (layer "F.Cu") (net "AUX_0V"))
 (segment (start 43.475 20) (end 43.475 20.54) (width 0.25) (layer "F.Cu") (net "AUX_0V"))
 (segment (start 41.775 13.5) (end 41.775 13.5) (width 0.25) (layer "F.Cu") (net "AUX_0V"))
 (segment (start 37.875 14.825) (end 38.875 14.825) (width 0.25) (layer "F.Cu") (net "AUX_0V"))
 (via (at 38.875 14.825) (size 0.6) (drill 0.3) (layers "F.Cu" "B.Cu") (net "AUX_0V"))
 (via (at 43.475 20.54) (size 0.6) (drill 0.3) (layers "F.Cu" "B.Cu") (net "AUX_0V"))
 (via (at 41.775 13.5) (size 0.6) (drill 0.3) (layers "F.Cu" "B.Cu") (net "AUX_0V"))
 (via (at 38.875 22.445) (size 0.6) (drill 0.3) (layers "F.Cu" "B.Cu") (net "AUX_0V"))
 (via (at 43.475 23) (size 0.6) (drill 0.3) (layers "F.Cu" "B.Cu") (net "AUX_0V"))
 (segment (start 37.875 19.905) (end 39 19.905) (width 0.25) (layer "F.Cu") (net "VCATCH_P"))
 (via (at 39 19.905) (size 0.6) (drill 0.3) (layers "F.Cu" "B.Cu") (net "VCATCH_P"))
 (segment (start 47 15) (end 53 15) (width 0.25) (layer "B.Cu") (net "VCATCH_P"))
 (segment (start 47 19.905) (end 47 15) (width 0.25) (layer "B.Cu") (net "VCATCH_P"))
 (segment (start 39 19.905) (end 47 19.905) (width 0.25) (layer "B.Cu") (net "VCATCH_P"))
 (segment (start 37.875 21.175) (end 39 21.175) (width 0.25) (layer "F.Cu") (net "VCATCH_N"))
 (via (at 39 21.175) (size 0.6) (drill 0.3) (layers "F.Cu" "B.Cu") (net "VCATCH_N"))
 (segment (start 48 21.175) (end 48 17.5) (width 0.25) (layer "B.Cu") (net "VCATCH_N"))
 (segment (start 48 17.5) (end 53 17.5) (width 0.25) (layer "B.Cu") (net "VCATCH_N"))
 (segment (start 39 21.175) (end 48 21.175) (width 0.25) (layer "B.Cu") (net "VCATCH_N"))
 (segment (start 44.825 27) (end 49 27) (width 0.25) (layer "F.Cu") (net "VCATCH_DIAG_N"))
 (segment (start 49 27) (end 49 20) (width 0.25) (layer "F.Cu") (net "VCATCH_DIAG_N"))
 (segment (start 46 27) (end 44.825 27) (width 0.25) (layer "F.Cu") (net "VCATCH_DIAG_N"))
 (segment (start 49 20) (end 53 20) (width 0.25) (layer "F.Cu") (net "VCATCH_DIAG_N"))
 (segment (start 46 16.094999) (end 46 27) (width 0.25) (layer "F.Cu") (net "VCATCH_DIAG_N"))
 (segment (start 37.875 16.094999) (end 38.7 16.094999) (width 0.25) (layer "F.Cu") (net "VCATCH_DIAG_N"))
 (via (at 46 16.094999) (size 0.6) (drill 0.3) (layers "F.Cu" "B.Cu") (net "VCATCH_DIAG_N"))
 (via (at 38.7 16.094999) (size 0.6) (drill 0.3) (layers "F.Cu" "B.Cu") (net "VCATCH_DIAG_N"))
 (segment (start 38.7 16.094999) (end 46 16.094999) (width 0.25) (layer "B.Cu") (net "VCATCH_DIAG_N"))
 (segment (start 25.4625 5) (end 25.4625 10) (width 0.25) (layer "F.Cu") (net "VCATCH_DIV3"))
 (segment (start 13.4625 5) (end 16.5375 5) (width 0.25) (layer "F.Cu") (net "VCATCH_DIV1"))
 (segment (start 19.4625 5) (end 22.5375 5) (width 0.25) (layer "F.Cu") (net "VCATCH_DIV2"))
 (segment (start 10.5375 10) (end 7.4625 10) (width 0.25) (layer "F.Cu") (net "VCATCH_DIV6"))
 (segment (start 4.5375 10) (end 4.5375 23) (width 0.25) (layer "F.Cu") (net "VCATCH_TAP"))
 (segment (start 17.5375 23) (end 17.5375 26) (width 0.25) (layer "F.Cu") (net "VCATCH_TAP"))
 (segment (start 28.125 19.905) (end 27 19.905) (width 0.25) (layer "F.Cu") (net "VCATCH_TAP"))
 (segment (start 17.5375 26) (end 18.225 26) (width 0.25) (layer "F.Cu") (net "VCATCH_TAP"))
 (segment (start 4.5375 23) (end 17.5375 23) (width 0.25) (layer "F.Cu") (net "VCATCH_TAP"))
 (via (at 27 19.905) (size 0.6) (drill 0.3) (layers "F.Cu" "B.Cu") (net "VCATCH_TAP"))
 (via (at 17.5375 23) (size 0.6) (drill 0.3) (layers "F.Cu" "B.Cu") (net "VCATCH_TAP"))
 (segment (start 17.5375 19.905) (end 17.5375 23) (width 0.25) (layer "B.Cu") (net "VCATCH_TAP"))
 (segment (start 27 19.905) (end 17.5375 19.905) (width 0.25) (layer "B.Cu") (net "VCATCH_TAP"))
 (segment (start 37.875 17.365) (end 39.5 17.365) (width 0.25) (layer "F.Cu") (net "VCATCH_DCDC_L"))
 (segment (start 39.5 17.365) (end 39.5 13.555) (width 0.25) (layer "F.Cu") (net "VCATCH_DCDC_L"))
 (segment (start 37.875 13.555) (end 40.225 13.555) (width 0.25) (layer "F.Cu") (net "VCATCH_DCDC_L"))
 (segment (start 40.225 13.555) (end 40.225 13.5) (width 0.25) (layer "F.Cu") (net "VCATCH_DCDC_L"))
 (segment (start 28.125 16.094999) (end 26.3 16.094999) (width 0.25) (layer "F.Cu") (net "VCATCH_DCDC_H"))
 (segment (start 26.3 13.555) (end 25.475 14) (width 0.25) (layer "F.Cu") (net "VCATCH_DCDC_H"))
 (segment (start 25.475 14) (end 25.475 16.5) (width 0.25) (layer "F.Cu") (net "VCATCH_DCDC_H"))
 (segment (start 28.125 13.555) (end 26.3 13.555) (width 0.25) (layer "F.Cu") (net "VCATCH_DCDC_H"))
 (segment (start 26.3 16.094999) (end 25.475 16.5) (width 0.25) (layer "F.Cu") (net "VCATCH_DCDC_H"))
 (segment (start 4.5375 3) (end 5.5375 5) (width 0.25) (layer "F.Cu") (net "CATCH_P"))
 (segment (start 3 3) (end 4.5375 3) (width 0.25) (layer "F.Cu") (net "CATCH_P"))
 (segment (start 8.4625 5) (end 10.5375 5) (width 0.25) (layer "F.Cu") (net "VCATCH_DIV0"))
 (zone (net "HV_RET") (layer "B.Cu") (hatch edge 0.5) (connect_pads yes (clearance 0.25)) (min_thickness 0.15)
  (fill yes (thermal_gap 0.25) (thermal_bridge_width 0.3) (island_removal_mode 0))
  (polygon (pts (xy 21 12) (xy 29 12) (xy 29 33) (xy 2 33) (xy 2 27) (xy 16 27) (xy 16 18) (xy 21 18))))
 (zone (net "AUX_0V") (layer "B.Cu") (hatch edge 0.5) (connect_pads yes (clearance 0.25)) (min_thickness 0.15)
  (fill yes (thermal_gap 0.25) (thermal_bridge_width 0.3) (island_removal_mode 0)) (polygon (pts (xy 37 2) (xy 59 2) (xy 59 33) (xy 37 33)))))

